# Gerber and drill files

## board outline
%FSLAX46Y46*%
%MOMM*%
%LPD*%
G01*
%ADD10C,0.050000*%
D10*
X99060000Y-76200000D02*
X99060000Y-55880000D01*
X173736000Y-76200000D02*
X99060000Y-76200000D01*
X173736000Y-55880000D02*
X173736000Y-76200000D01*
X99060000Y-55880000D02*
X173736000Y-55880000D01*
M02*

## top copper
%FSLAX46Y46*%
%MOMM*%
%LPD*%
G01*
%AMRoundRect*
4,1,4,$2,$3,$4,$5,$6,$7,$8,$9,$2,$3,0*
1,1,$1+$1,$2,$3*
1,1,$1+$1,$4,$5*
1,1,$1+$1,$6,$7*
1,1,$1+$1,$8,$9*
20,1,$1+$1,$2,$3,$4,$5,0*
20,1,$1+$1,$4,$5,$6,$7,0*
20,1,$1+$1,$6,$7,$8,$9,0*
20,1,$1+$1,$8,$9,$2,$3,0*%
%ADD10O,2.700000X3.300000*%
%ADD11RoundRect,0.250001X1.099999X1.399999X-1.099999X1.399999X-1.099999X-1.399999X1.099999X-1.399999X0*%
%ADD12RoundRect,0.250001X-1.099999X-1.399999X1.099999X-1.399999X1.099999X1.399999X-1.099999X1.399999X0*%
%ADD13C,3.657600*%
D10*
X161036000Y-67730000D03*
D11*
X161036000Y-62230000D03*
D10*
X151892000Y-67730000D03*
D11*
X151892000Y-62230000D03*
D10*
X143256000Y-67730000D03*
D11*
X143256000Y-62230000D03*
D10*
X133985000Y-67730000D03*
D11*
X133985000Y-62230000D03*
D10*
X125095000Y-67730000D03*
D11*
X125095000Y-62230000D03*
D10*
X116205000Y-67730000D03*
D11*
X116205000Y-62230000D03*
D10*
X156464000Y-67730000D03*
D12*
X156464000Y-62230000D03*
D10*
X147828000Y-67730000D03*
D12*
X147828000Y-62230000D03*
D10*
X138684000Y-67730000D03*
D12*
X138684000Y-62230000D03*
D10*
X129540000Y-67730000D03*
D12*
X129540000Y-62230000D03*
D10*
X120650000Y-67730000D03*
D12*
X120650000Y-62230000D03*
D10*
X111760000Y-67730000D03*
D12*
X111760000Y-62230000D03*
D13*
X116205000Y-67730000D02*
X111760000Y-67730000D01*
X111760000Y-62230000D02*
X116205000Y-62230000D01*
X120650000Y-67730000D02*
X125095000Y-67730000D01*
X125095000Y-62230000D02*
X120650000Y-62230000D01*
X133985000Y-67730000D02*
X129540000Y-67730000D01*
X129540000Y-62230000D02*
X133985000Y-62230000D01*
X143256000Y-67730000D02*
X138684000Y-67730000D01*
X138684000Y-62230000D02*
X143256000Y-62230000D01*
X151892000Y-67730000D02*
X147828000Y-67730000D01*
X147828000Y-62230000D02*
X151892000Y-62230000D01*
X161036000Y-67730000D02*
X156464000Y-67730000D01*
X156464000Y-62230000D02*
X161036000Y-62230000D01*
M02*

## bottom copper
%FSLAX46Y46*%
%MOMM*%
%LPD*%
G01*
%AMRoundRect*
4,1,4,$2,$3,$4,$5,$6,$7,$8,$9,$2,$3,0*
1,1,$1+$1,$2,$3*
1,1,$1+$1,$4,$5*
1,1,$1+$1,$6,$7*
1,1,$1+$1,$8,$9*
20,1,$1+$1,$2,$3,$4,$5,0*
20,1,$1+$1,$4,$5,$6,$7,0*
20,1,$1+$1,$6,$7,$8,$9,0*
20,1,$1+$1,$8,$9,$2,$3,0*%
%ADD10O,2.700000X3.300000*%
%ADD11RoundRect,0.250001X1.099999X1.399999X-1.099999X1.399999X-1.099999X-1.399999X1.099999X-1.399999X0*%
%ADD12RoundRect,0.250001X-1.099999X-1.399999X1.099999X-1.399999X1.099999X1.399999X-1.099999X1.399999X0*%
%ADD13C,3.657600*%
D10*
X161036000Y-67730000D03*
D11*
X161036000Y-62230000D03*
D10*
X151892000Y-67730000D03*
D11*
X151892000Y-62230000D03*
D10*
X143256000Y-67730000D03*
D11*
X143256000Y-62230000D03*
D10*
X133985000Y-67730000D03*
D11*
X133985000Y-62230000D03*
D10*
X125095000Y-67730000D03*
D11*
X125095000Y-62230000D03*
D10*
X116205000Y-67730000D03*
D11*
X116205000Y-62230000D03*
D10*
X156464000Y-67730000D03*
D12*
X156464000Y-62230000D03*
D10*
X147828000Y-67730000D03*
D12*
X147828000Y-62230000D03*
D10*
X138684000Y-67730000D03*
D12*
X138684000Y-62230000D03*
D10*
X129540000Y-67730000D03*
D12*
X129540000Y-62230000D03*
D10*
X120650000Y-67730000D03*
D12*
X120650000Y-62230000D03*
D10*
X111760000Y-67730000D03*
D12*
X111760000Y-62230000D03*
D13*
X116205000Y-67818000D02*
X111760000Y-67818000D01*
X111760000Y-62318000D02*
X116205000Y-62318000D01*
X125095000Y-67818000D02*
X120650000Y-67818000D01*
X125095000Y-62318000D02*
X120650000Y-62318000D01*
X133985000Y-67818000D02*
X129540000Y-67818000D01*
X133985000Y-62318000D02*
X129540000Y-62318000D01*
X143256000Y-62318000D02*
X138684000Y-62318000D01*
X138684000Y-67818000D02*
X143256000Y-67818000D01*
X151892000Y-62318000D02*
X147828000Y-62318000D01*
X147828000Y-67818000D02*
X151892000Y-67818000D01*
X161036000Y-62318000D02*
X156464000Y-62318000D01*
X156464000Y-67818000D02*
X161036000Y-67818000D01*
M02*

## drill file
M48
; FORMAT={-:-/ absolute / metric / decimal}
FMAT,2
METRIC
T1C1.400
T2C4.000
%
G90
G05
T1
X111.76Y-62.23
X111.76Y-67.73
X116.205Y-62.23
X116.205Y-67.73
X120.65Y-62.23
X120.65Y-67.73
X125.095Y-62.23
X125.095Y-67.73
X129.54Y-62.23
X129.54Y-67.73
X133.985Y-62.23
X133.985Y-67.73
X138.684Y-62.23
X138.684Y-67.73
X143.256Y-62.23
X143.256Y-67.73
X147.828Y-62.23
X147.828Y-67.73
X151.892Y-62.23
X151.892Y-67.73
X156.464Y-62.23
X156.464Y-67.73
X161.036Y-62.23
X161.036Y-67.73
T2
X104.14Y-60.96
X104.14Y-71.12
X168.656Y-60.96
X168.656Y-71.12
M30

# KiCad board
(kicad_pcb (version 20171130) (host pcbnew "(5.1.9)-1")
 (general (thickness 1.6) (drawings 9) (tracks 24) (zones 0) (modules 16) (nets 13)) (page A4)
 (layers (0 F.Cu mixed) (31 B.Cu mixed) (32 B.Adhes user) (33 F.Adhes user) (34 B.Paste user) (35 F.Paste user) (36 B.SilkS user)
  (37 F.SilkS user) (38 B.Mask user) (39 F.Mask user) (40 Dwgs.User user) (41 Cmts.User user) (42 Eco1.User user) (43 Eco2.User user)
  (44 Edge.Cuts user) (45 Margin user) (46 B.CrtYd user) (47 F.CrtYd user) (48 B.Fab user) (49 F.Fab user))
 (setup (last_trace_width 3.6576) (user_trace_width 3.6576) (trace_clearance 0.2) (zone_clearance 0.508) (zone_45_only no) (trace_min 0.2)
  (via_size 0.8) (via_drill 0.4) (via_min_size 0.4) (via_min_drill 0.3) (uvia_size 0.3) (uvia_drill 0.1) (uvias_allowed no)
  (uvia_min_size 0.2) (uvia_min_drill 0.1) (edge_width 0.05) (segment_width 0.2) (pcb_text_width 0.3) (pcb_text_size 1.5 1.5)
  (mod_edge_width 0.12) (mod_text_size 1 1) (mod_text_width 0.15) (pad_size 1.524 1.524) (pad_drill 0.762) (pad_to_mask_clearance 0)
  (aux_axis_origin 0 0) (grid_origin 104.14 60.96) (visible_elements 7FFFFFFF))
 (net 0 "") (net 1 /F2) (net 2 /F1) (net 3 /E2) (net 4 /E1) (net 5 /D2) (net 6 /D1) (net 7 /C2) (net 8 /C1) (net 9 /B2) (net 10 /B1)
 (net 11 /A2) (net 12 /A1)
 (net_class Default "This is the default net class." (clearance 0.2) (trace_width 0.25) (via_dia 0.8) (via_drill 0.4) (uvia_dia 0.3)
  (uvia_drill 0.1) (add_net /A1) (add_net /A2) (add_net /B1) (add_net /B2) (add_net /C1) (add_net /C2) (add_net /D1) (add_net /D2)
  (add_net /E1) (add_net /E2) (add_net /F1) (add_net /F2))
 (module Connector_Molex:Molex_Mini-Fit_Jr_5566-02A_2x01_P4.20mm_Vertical (layer B.Cu) (at 161.036 62.23 180)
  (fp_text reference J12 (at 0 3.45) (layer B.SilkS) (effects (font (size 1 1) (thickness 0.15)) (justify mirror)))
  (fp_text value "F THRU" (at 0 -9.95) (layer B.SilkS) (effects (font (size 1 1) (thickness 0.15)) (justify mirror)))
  (pad 2 thru_hole oval (at 0 -5.5 180) (size 2.7 3.3) (drill 1.4) (layers *.Cu *.Mask) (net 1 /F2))
  (pad 1 thru_hole roundrect (at 0 0 180) (size 2.7 3.3) (drill 1.4) (layers *.Cu *.Mask) (roundrect_rratio 0.09259299999999999) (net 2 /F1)))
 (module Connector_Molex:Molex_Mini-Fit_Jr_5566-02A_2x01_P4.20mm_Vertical (layer B.Cu) (at 151.892 62.23 180)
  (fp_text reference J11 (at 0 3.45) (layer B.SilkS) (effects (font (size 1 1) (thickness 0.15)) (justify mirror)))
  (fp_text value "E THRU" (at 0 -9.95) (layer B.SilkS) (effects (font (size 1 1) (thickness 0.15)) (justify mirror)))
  (pad 2 thru_hole oval (at 0 -5.5 180) (size 2.7 3.3) (drill 1.4) (layers *.Cu *.Mask) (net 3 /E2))
  (pad 1 thru_hole roundrect (at 0 0 180) (size 2.7 3.3) (drill 1.4) (layers *.Cu *.Mask) (roundrect_rratio 0.09259299999999999) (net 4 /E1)))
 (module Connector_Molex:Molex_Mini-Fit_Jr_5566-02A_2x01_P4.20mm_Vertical (layer B.Cu) (at 143.256 62.23 180)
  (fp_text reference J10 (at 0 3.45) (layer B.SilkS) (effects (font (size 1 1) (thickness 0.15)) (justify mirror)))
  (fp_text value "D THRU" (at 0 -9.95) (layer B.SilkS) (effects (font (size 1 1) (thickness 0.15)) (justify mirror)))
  (pad 2 thru_hole oval (at 0 -5.5 180) (size 2.7 3.3) (drill 1.4) (layers *.Cu *.Mask) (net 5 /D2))
  (pad 1 thru_hole roundrect (at 0 0 180) (size 2.7 3.3) (drill 1.4) (layers *.Cu *.Mask) (roundrect_rratio 0.09259299999999999) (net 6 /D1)))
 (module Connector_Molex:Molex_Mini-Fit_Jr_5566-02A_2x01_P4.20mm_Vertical (layer B.Cu) (at 133.985 62.23 180)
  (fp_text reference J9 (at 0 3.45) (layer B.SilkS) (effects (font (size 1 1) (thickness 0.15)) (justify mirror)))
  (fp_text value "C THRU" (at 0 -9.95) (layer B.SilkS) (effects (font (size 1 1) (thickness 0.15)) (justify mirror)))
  (pad 2 thru_hole oval (at 0 -5.5 180) (size 2.7 3.3) (drill 1.4) (layers *.Cu *.Mask) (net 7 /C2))
  (pad 1 thru_hole roundrect (at 0 0 180) (size 2.7 3.3) (drill 1.4) (layers *.Cu *.Mask) (roundrect_rratio 0.09259299999999999) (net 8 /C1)))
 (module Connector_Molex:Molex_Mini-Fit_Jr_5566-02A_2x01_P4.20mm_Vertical (layer B.Cu) (at 125.095 62.23 180)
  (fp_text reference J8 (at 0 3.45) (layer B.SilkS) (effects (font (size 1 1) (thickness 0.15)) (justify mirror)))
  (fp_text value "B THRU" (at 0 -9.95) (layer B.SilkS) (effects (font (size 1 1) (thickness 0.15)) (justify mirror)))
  (pad 2 thru_hole oval (at 0 -5.5 180) (size 2.7 3.3) (drill 1.4) (layers *.Cu *.Mask) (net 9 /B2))
  (pad 1 thru_hole roundrect (at 0 0 180) (size 2.7 3.3) (drill 1.4) (layers *.Cu *.Mask) (roundrect_rratio 0.09259299999999999)
   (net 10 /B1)))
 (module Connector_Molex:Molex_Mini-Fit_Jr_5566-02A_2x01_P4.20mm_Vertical (layer B.Cu) (at 116.205 62.23 180)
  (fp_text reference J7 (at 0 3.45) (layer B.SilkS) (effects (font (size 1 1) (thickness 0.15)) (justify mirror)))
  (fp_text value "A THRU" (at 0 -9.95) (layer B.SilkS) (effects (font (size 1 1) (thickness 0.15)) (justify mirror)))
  (pad 2 thru_hole oval (at 0 -5.5 180) (size 2.7 3.3) (drill 1.4) (layers *.Cu *.Mask) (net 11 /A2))
  (pad 1 thru_hole roundrect (at 0 0 180) (size 2.7 3.3) (drill 1.4) (layers *.Cu *.Mask) (roundrect_rratio 0.09259299999999999)
   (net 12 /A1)))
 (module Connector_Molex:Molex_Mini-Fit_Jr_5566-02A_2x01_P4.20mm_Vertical (layer F.Cu) (at 156.464 62.23)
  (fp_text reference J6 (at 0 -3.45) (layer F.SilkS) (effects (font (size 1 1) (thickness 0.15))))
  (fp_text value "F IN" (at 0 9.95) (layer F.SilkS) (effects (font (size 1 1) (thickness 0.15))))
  (pad 2 thru_hole oval (at 0 5.5) (size 2.7 3.3) (drill 1.4) (layers *.Cu *.Mask) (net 1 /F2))
  (pad 1 thru_hole roundrect (at 0 0) (size 2.7 3.3) (drill 1.4) (layers *.Cu *.Mask) (roundrect_rratio 0.09259299999999999) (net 2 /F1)))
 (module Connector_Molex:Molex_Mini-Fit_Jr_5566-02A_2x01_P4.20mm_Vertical (layer F.Cu) (at 147.828 62.23)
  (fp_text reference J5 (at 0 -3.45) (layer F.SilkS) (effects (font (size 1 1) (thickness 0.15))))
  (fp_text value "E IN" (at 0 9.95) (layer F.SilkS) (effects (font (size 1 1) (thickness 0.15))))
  (pad 2 thru_hole oval (at 0 5.5) (size 2.7 3.3) (drill 1.4) (layers *.Cu *.Mask) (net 3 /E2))
  (pad 1 thru_hole roundrect (at 0 0) (size 2.7 3.3) (drill 1.4) (layers *.Cu *.Mask) (roundrect_rratio 0.09259299999999999) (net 4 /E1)))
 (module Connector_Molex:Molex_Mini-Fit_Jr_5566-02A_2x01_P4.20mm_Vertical (layer F.Cu) (at 138.684 62.23)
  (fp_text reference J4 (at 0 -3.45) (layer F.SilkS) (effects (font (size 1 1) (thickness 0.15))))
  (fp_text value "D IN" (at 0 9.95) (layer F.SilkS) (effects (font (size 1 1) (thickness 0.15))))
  (pad 2 thru_hole oval (at 0 5.5) (size 2.7 3.3) (drill 1.4) (layers *.Cu *.Mask) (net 5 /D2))
  (pad 1 thru_hole roundrect (at 0 0) (size 2.7 3.3) (drill 1.4) (layers *.Cu *.Mask) (roundrect_rratio 0.09259299999999999) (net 6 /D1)))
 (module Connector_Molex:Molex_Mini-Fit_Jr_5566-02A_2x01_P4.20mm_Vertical (layer F.Cu) (at 129.54 62.23)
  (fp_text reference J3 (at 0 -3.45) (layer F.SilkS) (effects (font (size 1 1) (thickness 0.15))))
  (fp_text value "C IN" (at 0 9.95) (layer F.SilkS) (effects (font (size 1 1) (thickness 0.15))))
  (pad 2 thru_hole oval (at 0 5.5) (size 2.7 3.3) (drill 1.4) (layers *.Cu *.Mask) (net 7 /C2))
  (pad 1 thru_hole roundrect (at 0 0) (size 2.7 3.3) (drill 1.4) (layers *.Cu *.Mask) (roundrect_rratio 0.09259299999999999) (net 8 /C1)))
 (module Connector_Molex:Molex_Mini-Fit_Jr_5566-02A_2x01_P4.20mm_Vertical (layer F.Cu) (at 120.65 62.23)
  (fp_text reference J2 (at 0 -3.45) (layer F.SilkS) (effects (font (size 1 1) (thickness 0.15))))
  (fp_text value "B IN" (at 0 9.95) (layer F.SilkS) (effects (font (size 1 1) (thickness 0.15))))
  (pad 2 thru_hole oval (at 0 5.5) (size 2.7 3.3) (drill 1.4) (layers *.Cu *.Mask) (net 9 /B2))
  (pad 1 thru_hole roundrect (at 0 0) (size 2.7 3.3) (drill 1.4) (layers *.Cu *.Mask) (roundrect_rratio 0.09259299999999999) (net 10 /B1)))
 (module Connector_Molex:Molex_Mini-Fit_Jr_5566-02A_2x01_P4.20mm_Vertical (layer F.Cu) (at 111.76 62.23)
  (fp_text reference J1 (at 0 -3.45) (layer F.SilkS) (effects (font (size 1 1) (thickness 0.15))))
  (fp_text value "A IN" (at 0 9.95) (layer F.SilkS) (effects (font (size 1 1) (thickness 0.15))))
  (pad 2 thru_hole oval (at 0 5.5) (size 2.7 3.3) (drill 1.4) (layers *.Cu *.Mask) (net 11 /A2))
  (pad 1 thru_hole roundrect (at 0 0) (size 2.7 3.3) (drill 1.4) (layers *.Cu *.Mask) (roundrect_rratio 0.09259299999999999) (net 12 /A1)))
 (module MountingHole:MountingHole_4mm (layer F.Cu) (at 104.14 71.12)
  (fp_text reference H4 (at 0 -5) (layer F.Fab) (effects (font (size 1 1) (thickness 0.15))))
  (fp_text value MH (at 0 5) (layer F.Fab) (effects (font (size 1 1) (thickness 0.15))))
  (pad 1 np_thru_hole circle (at 0 0) (size 4 4) (drill 4) (layers *.Cu *.Mask)))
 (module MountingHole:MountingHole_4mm (layer F.Cu) (at 168.656 71.12)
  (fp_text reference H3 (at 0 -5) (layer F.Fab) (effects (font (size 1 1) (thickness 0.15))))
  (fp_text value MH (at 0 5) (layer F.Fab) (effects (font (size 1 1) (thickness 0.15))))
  (pad 1 np_thru_hole circle (at 0 0) (size 4 4) (drill 4) (layers *.Cu *.Mask)))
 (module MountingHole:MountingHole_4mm (layer F.Cu) (at 168.656 60.96)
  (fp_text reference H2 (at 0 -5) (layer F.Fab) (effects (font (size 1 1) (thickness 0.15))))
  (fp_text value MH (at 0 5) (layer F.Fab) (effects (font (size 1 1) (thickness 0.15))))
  (pad 1 np_thru_hole circle (at 0 0) (size 4 4) (drill 4) (layers *.Cu *.Mask)))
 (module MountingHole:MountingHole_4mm (layer F.Cu) (at 104.14 60.96)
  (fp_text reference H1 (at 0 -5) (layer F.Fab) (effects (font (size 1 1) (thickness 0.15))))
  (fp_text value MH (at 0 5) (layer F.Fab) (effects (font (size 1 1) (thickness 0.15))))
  (pad 1 np_thru_hole circle (at 0 0) (size 4 4) (drill 4) (layers *.Cu *.Mask)))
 (gr_line (start 99.06 76.2) (end 99.06 55.88) (layer Edge.Cuts) (width 0.05))
 (gr_line (start 173.736 76.2) (end 99.06 76.2) (layer Edge.Cuts) (width 0.05))
 (gr_line (start 173.736 55.88) (end 173.736 76.2) (layer Edge.Cuts) (width 0.05))
 (gr_line (start 99.06 55.88) (end 173.736 55.88) (layer Edge.Cuts) (width 0.05))
 (segment (start 116.205 67.73) (end 111.76 67.73) (width 3.6576) (layer F.Cu) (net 11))
 (segment (start 116.205 67.818) (end 111.76 67.818) (width 3.6576) (layer B.Cu) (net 11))
 (segment (start 111.76 62.23) (end 116.205 62.23) (width 3.6576) (layer F.Cu) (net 12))
 (segment (start 111.76 62.318) (end 116.205 62.318) (width 3.6576) (layer B.Cu) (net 12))
 (segment (start 120.65 67.73) (end 125.095 67.73) (width 3.6576) (layer F.Cu) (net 9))
 (segment (start 125.095 67.818) (end 120.65 67.818) (width 3.6576) (layer B.Cu) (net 9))
 (segment (start 125.095 62.23) (end 120.65 62.23) (width 3.6576) (layer F.Cu) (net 10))
 (segment (start 125.095 62.318) (end 120.65 62.318) (width 3.6576) (layer B.Cu) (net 10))
 (segment (start 133.985 67.73) (end 129.54 67.73) (width 3.6576) (layer F.Cu) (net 7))
 (segment (start 133.985 67.818) (end 129.54 67.818) (width 3.6576) (layer B.Cu) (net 7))
 (segment (start 129.54 62.23) (end 133.985 62.23) (width 3.6576) (layer F.Cu) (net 8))
 (segment (start 133.985 62.318) (end 129.54 62.318) (width 3.6576) (layer B.Cu) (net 8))
 (segment (start 143.256 67.73) (end 138.684 67.73) (width 3.6576) (layer F.Cu) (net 5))
 (segment (start 143.256 62.318) (end 138.684 62.318) (width 3.6576) (layer B.Cu) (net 6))
 (segment (start 138.684 62.23) (end 143.256 62.23) (width 3.6576) (layer F.Cu) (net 6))
 (segment (start 138.684 67.818) (end 143.256 67.818) (width 3.6576) (layer B.Cu) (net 5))
 (segment (start 151.892 67.73) (end 147.828 67.73) (width 3.6576) (layer F.Cu) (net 3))
 (segment (start 151.892 62.318) (end 147.828 62.318) (width 3.6576) (layer B.Cu) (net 4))
 (segment (start 147.828 62.23) (end 151.892 62.23) (width 3.6576) (layer F.Cu) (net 4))
 (segment (start 147.828 67.818) (end 151.892 67.818) (width 3.6576) (layer B.Cu) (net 3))
 (segment (start 161.036 67.73) (end 156.464 67.73) (width 3.6576) (layer F.Cu) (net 1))
 (segment (start 161.036 62.318) (end 156.464 62.318) (width 3.6576) (layer B.Cu) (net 2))
 (segment (start 156.464 62.23) (end 161.036 62.23) (width 3.6576) (layer F.Cu) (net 2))
 (segment (start 156.464 67.818) (end 161.036 67.818) (width 3.6576) (layer B.Cu) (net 1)))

